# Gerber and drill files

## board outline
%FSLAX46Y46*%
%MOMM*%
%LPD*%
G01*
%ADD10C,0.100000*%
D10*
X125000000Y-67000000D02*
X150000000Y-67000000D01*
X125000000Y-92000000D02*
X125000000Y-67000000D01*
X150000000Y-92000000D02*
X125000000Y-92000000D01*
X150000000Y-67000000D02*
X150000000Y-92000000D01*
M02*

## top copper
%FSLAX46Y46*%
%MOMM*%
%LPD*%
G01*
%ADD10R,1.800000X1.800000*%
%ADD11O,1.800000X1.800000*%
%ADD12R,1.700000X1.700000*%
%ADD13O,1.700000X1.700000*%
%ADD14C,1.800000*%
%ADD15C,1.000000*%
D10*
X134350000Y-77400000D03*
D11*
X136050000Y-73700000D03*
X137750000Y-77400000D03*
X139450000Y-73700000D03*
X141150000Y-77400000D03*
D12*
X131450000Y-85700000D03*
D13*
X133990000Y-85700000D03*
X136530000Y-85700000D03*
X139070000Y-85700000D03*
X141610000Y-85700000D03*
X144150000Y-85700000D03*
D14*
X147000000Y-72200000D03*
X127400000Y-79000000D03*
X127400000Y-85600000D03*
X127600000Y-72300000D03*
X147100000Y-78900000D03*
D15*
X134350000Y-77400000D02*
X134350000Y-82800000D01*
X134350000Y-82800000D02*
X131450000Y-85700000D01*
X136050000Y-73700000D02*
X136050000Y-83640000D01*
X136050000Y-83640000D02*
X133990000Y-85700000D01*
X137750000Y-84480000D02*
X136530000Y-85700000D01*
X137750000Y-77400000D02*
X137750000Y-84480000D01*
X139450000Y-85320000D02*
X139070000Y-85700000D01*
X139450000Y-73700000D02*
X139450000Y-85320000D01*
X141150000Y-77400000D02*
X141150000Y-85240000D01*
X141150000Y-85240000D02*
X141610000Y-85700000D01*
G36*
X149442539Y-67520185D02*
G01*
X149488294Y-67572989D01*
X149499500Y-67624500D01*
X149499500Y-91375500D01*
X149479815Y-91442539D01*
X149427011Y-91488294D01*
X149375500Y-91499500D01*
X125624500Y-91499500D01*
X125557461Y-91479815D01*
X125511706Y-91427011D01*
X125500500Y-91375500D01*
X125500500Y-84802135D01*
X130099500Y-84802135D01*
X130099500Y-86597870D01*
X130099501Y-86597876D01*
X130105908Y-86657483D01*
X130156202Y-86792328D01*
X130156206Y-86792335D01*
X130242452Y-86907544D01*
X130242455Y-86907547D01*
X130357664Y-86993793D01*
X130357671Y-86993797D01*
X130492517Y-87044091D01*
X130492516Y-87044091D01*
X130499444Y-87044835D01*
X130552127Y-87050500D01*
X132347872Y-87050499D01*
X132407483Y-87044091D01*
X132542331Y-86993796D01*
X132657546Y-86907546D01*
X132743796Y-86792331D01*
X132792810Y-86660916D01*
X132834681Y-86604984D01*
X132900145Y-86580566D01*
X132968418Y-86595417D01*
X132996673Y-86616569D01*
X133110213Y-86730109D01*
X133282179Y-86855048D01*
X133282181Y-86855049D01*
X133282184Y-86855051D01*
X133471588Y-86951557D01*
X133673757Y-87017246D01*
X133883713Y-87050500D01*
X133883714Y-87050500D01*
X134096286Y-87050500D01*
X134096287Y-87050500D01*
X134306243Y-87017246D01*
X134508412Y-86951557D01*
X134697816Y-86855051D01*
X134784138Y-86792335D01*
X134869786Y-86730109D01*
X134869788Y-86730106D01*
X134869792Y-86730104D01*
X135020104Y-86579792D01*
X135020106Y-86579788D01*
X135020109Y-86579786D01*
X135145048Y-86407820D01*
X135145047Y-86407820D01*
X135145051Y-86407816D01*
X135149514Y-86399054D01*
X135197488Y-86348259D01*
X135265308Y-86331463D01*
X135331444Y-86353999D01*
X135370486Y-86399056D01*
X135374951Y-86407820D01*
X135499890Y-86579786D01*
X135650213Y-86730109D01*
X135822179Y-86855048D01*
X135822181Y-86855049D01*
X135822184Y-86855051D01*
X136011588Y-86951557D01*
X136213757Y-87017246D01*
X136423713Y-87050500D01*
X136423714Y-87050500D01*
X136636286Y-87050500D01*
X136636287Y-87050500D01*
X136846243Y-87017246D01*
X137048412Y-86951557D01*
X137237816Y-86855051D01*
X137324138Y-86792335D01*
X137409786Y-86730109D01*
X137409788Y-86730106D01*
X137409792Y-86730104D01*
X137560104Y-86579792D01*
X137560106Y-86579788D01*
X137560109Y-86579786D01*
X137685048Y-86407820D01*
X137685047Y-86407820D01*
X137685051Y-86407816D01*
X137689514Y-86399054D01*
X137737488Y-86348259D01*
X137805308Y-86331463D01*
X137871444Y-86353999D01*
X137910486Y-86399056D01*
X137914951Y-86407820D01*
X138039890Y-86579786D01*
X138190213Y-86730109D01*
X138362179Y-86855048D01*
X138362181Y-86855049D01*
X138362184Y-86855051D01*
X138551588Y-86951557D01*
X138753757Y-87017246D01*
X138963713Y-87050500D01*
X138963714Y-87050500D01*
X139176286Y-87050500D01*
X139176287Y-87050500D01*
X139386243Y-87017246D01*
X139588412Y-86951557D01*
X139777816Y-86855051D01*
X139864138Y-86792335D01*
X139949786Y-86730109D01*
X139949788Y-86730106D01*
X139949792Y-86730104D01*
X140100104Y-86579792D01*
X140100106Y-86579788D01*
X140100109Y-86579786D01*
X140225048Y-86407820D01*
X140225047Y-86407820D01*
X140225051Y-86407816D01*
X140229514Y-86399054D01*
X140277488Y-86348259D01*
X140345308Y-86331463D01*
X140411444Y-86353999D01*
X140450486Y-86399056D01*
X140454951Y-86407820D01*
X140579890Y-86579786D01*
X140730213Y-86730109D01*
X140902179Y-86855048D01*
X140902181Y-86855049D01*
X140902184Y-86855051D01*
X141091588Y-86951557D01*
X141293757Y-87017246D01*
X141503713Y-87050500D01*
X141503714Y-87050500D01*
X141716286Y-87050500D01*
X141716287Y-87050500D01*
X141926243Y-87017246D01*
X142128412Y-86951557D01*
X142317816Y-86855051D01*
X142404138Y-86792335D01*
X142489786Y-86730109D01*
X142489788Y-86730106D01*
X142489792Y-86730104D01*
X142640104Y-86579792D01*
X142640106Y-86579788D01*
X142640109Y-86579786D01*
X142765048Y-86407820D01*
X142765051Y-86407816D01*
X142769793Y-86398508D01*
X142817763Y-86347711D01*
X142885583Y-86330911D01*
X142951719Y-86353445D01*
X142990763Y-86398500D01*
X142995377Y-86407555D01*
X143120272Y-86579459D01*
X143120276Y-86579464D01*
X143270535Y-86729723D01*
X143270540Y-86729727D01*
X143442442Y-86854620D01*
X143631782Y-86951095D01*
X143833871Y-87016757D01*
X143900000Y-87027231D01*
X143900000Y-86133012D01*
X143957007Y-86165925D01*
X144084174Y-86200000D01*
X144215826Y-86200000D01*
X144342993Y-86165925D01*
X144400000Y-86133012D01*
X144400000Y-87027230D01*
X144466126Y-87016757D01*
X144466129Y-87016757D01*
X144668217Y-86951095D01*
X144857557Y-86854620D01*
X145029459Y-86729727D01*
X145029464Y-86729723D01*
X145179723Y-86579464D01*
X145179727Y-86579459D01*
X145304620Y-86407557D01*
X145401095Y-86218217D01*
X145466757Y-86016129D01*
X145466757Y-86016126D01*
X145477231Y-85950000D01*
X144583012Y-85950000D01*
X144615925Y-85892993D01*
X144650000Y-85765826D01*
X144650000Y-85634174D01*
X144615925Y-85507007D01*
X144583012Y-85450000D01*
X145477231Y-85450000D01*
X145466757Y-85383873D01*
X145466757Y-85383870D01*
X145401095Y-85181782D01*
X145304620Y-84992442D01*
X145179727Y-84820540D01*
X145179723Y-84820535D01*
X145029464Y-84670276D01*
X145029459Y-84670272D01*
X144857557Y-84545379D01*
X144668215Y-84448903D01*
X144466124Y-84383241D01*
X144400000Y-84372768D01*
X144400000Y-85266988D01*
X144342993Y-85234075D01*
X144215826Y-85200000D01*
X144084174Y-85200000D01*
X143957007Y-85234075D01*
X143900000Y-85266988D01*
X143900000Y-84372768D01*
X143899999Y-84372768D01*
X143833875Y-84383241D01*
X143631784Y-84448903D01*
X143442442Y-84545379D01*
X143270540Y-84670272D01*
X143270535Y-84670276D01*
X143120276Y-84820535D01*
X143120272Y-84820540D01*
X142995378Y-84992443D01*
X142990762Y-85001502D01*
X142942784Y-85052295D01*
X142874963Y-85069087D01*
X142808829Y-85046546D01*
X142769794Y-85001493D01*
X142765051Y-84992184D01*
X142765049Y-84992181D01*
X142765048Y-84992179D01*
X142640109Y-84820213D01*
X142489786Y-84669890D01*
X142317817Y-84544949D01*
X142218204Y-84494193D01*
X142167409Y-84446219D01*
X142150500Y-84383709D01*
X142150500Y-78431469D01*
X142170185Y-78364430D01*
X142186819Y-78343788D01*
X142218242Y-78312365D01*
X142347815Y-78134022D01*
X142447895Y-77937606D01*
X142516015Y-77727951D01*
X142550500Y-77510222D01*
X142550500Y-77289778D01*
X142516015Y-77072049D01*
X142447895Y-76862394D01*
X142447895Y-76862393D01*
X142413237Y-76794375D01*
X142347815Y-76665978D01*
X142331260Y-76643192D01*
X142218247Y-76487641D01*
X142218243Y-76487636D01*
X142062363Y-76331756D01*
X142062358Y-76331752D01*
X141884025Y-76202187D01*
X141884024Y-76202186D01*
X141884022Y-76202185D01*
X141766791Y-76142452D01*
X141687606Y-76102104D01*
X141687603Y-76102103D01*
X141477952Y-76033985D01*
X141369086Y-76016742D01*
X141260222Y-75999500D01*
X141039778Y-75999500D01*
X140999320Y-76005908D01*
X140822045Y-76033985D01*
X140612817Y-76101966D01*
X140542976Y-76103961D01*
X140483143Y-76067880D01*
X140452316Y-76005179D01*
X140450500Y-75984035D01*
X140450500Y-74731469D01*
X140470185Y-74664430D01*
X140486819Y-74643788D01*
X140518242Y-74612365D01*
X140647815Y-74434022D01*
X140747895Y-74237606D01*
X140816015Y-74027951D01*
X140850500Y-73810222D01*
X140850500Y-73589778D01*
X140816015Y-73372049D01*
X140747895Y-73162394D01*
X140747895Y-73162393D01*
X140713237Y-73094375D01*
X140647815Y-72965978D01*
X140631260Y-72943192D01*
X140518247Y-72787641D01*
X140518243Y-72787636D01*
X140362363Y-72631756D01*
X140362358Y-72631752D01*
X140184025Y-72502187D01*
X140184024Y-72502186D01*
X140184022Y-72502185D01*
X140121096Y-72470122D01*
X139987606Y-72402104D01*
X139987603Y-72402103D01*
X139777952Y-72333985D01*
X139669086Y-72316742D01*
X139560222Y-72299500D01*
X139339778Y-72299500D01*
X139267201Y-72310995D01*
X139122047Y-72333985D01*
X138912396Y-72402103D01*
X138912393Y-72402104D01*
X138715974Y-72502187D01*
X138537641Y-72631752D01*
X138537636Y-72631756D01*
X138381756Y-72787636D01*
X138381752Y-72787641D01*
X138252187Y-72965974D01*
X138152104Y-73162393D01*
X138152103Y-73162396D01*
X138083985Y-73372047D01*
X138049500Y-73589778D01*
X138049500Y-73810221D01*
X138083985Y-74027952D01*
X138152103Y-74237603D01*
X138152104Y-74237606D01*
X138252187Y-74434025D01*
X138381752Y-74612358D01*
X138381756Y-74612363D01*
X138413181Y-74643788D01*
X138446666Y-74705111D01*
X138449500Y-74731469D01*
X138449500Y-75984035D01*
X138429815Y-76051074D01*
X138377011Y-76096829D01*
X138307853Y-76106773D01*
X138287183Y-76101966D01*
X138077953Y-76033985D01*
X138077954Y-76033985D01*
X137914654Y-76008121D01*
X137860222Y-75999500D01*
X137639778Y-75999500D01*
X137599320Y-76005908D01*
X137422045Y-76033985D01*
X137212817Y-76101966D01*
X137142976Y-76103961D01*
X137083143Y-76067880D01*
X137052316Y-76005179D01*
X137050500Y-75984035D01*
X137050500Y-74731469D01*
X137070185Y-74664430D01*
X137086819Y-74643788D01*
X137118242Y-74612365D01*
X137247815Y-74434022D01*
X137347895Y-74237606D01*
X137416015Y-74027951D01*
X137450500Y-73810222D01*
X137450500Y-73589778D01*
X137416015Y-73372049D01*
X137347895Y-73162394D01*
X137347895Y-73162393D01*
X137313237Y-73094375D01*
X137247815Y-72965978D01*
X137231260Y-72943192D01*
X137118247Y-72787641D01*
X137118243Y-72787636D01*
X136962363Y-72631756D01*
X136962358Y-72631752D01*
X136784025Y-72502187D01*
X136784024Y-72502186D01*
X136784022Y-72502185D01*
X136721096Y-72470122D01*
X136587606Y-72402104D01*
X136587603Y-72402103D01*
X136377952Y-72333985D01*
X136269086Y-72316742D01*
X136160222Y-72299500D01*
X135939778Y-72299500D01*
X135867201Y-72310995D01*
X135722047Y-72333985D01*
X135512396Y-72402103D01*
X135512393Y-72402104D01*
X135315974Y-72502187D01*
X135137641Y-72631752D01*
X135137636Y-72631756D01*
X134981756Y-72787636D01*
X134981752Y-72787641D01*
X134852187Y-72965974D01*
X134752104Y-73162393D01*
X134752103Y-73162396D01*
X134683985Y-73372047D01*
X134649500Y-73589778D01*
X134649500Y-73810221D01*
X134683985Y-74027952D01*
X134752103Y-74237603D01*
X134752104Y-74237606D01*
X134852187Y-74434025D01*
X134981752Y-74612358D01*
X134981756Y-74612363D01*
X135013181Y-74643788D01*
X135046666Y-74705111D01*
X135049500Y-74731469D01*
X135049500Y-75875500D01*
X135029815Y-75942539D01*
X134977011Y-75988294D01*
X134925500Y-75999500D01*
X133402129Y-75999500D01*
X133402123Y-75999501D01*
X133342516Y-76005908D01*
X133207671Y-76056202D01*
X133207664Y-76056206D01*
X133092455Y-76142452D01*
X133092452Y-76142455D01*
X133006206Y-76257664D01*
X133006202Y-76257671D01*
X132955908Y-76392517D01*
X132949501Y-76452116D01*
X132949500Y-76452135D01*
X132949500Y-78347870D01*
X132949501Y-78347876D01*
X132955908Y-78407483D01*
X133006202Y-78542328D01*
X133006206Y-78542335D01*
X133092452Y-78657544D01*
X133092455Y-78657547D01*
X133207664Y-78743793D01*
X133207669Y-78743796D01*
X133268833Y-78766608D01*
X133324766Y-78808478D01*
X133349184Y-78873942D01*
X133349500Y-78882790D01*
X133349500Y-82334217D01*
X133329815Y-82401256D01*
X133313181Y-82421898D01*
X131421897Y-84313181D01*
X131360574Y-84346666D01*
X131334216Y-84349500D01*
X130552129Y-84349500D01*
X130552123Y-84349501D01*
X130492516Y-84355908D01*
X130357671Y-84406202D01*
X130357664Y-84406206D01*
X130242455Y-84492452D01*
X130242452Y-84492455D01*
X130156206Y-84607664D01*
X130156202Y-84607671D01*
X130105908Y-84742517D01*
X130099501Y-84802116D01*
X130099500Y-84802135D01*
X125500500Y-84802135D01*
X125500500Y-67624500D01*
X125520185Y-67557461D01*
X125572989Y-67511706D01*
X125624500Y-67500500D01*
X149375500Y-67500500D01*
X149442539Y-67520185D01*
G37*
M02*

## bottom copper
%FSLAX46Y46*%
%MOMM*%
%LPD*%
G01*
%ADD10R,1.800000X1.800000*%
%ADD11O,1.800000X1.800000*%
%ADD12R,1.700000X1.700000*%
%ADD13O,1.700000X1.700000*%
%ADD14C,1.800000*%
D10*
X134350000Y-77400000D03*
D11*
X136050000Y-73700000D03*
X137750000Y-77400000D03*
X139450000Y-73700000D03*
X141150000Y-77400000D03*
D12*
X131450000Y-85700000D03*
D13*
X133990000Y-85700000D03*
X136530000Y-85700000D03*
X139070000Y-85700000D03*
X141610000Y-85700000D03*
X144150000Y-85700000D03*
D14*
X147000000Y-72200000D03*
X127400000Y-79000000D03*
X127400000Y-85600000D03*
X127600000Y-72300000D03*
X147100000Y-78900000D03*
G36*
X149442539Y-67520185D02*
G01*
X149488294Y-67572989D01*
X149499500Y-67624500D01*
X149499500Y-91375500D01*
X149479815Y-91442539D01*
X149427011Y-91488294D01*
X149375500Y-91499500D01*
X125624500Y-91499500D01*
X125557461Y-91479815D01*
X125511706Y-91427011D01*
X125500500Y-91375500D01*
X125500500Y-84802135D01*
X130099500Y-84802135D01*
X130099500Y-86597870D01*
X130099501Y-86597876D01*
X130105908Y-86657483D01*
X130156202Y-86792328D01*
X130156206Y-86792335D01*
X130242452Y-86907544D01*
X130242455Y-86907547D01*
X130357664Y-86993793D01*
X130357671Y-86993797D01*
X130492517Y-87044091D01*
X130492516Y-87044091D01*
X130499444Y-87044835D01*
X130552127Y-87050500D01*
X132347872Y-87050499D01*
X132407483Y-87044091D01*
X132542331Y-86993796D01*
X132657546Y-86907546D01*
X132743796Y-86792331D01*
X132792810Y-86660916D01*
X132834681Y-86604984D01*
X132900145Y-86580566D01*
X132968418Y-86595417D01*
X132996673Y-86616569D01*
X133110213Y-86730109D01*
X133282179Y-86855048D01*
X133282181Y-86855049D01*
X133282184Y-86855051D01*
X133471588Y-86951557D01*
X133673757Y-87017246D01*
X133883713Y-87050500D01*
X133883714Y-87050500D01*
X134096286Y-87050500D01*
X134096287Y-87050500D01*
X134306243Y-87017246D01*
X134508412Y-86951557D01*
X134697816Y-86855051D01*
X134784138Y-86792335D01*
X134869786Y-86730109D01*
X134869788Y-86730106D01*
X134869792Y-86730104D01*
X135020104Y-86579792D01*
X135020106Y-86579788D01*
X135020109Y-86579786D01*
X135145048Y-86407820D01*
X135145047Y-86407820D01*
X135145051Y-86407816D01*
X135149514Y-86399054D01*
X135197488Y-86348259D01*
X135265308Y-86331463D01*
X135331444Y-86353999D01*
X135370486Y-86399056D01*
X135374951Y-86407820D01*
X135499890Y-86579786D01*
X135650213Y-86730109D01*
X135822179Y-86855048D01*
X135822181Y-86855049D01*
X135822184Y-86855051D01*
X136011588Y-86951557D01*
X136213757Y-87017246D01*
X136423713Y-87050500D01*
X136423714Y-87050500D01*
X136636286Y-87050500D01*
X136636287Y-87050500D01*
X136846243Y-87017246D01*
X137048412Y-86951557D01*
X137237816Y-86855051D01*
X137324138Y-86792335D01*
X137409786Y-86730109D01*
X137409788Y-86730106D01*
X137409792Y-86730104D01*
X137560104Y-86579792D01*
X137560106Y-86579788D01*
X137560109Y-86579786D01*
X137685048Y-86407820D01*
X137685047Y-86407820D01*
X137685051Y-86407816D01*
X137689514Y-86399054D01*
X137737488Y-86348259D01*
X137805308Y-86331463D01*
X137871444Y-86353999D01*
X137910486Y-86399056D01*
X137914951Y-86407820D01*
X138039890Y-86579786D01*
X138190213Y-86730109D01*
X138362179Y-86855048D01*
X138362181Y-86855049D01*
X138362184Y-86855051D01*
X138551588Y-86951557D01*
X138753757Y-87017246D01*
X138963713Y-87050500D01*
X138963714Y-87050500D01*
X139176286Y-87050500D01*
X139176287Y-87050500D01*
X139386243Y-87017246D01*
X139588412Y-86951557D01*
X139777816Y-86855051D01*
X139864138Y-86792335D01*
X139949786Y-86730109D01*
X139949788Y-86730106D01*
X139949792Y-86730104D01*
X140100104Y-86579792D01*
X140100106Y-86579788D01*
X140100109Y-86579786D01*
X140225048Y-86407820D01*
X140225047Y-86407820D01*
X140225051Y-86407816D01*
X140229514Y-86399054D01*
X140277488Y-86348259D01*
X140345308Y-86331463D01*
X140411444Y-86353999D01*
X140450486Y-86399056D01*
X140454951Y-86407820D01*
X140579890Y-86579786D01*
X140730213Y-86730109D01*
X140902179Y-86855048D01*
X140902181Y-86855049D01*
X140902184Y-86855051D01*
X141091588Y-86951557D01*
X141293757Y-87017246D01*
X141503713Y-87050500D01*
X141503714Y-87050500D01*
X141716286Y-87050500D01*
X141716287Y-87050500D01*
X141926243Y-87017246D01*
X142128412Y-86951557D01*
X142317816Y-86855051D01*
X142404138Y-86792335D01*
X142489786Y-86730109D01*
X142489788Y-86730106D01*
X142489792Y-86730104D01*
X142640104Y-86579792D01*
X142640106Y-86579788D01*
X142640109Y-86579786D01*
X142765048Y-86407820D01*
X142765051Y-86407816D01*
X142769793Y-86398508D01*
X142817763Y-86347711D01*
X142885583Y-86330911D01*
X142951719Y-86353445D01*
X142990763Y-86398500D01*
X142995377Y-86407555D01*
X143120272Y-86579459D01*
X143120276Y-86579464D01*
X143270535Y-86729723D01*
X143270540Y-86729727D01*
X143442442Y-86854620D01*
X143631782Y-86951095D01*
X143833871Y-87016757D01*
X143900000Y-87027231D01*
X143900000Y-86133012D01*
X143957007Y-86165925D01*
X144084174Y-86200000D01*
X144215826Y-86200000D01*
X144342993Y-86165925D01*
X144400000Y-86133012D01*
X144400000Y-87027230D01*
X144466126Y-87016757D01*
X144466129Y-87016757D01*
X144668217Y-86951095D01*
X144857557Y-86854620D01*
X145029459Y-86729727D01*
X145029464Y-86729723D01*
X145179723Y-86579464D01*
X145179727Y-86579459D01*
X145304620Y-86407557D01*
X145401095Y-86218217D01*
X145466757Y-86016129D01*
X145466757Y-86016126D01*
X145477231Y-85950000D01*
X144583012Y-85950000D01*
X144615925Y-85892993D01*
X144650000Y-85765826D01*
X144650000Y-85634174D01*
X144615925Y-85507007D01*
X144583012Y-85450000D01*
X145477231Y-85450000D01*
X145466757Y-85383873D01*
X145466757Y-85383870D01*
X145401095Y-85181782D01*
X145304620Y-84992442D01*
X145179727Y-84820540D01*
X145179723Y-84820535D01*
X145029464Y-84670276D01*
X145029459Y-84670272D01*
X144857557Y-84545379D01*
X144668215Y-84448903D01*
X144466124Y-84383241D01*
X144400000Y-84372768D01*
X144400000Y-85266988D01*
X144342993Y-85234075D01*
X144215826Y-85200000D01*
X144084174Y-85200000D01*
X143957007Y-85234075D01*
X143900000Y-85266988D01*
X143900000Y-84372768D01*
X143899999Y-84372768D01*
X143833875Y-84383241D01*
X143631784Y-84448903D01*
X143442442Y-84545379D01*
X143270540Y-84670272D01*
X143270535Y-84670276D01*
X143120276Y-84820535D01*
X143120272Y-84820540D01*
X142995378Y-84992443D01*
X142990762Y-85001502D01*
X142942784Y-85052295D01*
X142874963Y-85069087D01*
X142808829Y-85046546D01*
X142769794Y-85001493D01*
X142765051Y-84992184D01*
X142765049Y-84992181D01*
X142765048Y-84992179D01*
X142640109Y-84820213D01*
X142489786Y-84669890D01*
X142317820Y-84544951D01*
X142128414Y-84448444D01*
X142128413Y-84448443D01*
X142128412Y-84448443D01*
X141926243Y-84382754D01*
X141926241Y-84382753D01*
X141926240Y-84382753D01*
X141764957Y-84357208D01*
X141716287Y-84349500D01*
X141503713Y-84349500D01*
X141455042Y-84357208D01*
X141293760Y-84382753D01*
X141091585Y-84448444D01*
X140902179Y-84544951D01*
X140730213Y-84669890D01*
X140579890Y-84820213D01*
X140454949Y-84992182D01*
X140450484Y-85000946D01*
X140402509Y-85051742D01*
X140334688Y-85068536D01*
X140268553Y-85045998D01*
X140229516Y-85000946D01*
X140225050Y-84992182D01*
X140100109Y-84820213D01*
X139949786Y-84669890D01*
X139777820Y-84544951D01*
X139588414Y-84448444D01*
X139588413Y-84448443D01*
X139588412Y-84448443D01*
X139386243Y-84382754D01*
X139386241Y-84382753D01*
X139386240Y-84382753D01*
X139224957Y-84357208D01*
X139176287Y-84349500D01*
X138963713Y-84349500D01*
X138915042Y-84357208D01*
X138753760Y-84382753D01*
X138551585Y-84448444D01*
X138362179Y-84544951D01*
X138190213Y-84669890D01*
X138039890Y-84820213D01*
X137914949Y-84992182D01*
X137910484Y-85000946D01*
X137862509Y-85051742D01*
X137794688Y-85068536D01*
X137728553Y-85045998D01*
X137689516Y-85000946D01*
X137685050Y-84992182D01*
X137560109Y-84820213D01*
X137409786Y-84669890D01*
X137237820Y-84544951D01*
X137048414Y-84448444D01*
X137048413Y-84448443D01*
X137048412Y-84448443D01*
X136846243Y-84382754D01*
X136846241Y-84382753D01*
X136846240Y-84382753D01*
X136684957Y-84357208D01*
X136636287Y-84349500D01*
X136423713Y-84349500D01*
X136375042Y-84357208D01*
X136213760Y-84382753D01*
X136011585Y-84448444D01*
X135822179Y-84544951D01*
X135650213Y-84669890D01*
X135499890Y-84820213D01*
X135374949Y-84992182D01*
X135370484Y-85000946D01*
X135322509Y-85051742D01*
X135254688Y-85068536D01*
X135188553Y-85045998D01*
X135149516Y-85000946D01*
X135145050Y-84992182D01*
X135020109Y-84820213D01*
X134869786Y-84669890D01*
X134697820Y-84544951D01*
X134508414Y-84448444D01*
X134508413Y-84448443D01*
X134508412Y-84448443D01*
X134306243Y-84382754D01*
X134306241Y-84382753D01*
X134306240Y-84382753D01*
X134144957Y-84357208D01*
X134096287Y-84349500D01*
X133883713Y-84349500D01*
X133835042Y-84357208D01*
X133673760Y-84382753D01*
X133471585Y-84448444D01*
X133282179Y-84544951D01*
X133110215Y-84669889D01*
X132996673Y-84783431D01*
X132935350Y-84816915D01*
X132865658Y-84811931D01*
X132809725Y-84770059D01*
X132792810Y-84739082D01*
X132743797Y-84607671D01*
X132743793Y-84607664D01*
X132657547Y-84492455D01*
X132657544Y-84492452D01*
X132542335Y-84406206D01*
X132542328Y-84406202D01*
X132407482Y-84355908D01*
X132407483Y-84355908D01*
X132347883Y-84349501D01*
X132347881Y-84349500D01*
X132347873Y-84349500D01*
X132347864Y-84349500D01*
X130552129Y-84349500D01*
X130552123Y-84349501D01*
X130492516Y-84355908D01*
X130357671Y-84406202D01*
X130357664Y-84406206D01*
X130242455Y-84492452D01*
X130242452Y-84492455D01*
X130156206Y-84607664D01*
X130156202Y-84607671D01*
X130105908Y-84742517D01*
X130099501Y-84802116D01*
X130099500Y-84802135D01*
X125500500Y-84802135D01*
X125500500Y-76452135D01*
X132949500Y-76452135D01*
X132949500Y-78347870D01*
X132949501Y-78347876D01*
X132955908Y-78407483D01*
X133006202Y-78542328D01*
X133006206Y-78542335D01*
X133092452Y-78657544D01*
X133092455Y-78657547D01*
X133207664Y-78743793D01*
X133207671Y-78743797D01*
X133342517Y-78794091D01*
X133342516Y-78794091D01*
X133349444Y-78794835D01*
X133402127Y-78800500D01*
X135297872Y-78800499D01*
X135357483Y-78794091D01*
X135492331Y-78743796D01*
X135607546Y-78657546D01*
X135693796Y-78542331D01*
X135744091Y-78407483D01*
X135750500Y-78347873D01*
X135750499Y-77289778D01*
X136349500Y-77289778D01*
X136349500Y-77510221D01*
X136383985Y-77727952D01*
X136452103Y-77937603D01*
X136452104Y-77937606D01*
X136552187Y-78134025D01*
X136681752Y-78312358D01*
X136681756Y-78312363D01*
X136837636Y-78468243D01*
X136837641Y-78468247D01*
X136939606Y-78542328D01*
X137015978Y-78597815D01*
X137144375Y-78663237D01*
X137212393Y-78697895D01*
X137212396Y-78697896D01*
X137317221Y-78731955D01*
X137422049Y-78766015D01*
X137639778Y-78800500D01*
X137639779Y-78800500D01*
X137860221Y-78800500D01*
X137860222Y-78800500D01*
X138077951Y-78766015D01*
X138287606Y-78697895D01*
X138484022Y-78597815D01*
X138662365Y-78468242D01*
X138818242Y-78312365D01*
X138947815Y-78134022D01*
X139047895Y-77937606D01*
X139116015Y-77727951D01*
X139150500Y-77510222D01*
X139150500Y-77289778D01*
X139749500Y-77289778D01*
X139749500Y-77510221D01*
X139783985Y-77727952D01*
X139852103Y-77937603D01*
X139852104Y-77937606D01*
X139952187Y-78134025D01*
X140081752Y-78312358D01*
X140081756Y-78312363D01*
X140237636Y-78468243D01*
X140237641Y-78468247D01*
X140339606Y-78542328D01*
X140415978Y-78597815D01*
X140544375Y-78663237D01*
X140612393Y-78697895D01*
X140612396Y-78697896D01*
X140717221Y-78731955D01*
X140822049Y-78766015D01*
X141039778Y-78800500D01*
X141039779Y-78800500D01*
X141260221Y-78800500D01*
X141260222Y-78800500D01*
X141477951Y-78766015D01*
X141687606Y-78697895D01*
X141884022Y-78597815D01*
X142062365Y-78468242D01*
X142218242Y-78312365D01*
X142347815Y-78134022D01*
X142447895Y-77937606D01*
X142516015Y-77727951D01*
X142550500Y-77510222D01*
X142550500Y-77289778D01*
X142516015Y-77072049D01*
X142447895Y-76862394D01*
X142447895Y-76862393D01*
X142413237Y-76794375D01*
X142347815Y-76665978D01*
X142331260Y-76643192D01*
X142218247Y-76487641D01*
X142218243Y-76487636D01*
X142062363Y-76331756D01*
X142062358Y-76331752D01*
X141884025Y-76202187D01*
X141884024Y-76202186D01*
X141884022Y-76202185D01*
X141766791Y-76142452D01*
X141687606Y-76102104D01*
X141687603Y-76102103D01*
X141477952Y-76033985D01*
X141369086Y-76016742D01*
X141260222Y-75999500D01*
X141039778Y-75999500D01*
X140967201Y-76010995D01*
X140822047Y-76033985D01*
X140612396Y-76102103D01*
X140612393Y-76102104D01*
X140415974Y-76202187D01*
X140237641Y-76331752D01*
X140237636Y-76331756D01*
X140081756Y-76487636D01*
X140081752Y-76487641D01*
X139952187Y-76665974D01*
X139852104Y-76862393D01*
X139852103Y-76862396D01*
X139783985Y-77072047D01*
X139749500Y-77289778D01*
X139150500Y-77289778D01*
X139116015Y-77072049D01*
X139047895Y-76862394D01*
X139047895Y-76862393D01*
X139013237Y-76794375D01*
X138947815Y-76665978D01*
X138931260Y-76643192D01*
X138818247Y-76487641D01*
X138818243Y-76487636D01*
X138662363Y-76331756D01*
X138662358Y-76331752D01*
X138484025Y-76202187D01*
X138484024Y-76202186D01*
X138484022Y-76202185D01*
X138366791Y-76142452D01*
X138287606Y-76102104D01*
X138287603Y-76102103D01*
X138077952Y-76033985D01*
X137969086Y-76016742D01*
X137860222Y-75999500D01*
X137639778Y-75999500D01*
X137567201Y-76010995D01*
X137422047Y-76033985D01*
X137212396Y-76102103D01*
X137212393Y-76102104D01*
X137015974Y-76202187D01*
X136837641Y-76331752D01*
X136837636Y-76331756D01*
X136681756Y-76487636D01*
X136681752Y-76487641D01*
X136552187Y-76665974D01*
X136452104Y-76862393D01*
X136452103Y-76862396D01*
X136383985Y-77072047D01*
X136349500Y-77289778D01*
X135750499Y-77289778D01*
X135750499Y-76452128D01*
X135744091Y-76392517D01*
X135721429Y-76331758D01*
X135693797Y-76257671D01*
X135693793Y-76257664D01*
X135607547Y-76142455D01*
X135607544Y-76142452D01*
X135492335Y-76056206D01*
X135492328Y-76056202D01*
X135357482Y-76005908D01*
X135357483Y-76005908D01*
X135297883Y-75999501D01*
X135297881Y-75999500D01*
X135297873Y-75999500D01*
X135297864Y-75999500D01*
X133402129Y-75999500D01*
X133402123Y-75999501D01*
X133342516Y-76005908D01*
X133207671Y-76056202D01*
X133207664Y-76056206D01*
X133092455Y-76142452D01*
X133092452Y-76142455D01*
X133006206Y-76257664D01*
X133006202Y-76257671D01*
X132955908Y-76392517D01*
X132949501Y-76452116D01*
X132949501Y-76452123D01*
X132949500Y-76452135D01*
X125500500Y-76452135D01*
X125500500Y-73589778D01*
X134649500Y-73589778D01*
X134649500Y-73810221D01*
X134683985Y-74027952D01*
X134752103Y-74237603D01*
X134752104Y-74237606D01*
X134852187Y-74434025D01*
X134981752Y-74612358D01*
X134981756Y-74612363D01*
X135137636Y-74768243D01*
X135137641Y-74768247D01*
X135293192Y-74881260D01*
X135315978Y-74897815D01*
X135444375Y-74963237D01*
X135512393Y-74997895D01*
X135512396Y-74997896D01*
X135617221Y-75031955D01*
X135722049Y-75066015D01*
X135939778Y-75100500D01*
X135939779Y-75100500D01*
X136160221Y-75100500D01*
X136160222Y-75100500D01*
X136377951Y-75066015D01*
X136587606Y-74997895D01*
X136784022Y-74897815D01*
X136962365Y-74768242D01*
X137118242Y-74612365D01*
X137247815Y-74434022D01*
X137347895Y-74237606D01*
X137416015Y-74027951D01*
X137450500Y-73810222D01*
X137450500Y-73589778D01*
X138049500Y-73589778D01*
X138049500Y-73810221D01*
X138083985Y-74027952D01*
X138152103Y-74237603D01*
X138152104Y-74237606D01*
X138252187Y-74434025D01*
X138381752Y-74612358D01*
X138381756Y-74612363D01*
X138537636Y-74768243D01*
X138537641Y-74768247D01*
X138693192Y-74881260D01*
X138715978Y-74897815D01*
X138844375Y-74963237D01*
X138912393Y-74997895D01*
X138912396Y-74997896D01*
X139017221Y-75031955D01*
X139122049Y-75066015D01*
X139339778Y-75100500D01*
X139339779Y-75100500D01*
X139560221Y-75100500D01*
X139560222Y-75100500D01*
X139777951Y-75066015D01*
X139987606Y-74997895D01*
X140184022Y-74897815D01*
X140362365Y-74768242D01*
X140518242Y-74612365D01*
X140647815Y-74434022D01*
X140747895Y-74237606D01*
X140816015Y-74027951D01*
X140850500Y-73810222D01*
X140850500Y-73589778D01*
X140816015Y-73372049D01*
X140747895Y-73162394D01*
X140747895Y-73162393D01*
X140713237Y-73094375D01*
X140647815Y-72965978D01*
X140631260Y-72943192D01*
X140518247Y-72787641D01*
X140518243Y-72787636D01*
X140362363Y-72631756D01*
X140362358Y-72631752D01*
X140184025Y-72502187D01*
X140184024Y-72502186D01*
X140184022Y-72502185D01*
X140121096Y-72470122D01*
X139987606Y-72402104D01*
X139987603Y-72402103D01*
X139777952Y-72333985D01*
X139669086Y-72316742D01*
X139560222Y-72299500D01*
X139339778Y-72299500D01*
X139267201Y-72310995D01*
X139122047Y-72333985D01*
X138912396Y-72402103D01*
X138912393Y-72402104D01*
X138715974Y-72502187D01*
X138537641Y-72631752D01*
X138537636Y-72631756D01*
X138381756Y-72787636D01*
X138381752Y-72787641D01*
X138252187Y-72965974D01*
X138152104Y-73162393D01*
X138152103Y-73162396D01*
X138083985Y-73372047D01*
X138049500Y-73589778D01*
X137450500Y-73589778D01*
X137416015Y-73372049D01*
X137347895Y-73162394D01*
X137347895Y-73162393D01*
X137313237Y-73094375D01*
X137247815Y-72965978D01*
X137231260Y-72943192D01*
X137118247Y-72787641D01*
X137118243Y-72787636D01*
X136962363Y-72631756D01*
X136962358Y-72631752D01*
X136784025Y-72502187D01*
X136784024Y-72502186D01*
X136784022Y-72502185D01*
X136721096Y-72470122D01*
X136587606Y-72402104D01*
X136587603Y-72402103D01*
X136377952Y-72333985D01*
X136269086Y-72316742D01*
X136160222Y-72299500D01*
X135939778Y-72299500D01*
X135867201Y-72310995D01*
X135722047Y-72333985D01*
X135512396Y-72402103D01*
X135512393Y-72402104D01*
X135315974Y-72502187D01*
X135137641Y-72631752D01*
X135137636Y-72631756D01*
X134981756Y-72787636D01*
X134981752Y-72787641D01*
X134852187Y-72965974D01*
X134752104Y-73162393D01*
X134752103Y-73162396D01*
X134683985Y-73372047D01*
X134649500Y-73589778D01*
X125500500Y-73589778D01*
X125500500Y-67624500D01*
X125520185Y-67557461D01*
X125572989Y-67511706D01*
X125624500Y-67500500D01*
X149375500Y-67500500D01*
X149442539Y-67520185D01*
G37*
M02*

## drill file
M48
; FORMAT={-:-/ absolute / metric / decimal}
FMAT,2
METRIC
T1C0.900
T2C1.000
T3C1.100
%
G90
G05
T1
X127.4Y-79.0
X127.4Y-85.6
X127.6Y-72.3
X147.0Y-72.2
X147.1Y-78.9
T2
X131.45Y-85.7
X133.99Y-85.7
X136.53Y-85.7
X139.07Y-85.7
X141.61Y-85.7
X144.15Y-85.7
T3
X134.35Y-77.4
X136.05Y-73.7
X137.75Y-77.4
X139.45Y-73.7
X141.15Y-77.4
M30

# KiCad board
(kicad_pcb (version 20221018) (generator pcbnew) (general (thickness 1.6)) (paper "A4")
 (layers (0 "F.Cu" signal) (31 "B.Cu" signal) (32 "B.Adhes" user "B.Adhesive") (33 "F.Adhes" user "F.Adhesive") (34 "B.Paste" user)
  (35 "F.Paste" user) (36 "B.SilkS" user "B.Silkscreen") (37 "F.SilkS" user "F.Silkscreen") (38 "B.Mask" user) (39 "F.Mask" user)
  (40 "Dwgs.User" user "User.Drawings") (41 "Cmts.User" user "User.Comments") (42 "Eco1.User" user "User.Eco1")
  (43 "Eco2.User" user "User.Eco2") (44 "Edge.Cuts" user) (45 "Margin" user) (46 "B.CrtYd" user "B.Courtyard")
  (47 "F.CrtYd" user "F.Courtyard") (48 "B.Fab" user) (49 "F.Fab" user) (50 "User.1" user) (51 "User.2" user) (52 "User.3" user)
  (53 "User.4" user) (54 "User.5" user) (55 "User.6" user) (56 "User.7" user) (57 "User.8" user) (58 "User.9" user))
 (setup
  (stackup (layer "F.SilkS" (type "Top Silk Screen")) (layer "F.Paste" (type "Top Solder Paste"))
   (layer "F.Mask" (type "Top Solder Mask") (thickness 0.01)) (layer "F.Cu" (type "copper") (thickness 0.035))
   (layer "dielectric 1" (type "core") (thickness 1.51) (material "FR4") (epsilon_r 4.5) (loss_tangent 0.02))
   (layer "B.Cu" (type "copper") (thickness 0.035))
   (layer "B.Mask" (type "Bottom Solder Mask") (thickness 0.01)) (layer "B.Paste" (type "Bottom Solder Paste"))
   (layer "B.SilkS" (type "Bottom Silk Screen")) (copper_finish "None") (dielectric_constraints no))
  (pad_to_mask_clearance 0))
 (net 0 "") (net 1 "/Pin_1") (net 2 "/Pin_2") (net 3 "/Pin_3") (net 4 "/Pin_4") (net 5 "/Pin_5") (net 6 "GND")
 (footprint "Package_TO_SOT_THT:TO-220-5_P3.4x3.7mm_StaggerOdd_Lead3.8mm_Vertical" (layer "F.Cu") (at 134.35 77.4)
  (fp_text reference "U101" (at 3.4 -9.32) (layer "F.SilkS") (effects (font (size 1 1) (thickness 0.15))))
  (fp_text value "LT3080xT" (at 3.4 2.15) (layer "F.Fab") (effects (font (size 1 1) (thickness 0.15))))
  (pad "1" thru_hole rect (at 0 0) (size 1.8 1.8) (drill 1.1) (layers "*.Cu" "*.Mask") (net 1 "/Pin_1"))
  (pad "2" thru_hole oval (at 1.7 -3.7) (size 1.8 1.8) (drill 1.1) (layers "*.Cu" "*.Mask") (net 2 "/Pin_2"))
  (pad "3" thru_hole oval (at 3.4 0) (size 1.8 1.8) (drill 1.1) (layers "*.Cu" "*.Mask") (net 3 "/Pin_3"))
  (pad "4" thru_hole oval (at 5.1 -3.7) (size 1.8 1.8) (drill 1.1) (layers "*.Cu" "*.Mask") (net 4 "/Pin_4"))
  (pad "5" thru_hole oval (at 6.8 0) (size 1.8 1.8) (drill 1.1) (layers "*.Cu" "*.Mask") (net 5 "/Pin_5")))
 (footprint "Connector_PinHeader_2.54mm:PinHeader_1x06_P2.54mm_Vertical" (layer "B.Cu") (at 131.45 85.7 -90)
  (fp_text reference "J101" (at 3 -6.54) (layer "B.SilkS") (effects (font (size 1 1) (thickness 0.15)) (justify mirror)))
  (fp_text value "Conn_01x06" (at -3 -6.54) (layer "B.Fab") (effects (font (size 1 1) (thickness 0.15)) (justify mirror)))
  (pad "1" thru_hole rect (at 0 0 270) (size 1.7 1.7) (drill 1) (layers "*.Cu" "*.Mask") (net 1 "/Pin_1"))
  (pad "2" thru_hole oval (at 0 -2.54 270) (size 1.7 1.7) (drill 1) (layers "*.Cu" "*.Mask") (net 2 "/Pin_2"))
  (pad "3" thru_hole oval (at 0 -5.08 270) (size 1.7 1.7) (drill 1) (layers "*.Cu" "*.Mask") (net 3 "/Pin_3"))
  (pad "4" thru_hole oval (at 0 -7.62 270) (size 1.7 1.7) (drill 1) (layers "*.Cu" "*.Mask") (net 4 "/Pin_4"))
  (pad "5" thru_hole oval (at 0 -10.16 270) (size 1.7 1.7) (drill 1) (layers "*.Cu" "*.Mask") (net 5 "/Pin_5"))
  (pad "6" thru_hole oval (at 0 -12.7 270) (size 1.7 1.7) (drill 1) (layers "*.Cu" "*.Mask") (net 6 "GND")))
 (gr_line (start 125 67) (end 150 67) (stroke (width 0.1) (type default)) (layer "Edge.Cuts"))
 (gr_line (start 125 92) (end 125 67) (stroke (width 0.1) (type default)) (layer "Edge.Cuts"))
 (gr_line (start 150 92) (end 125 92) (stroke (width 0.1) (type default)) (layer "Edge.Cuts"))
 (gr_line (start 150 67) (end 150 92) (stroke (width 0.1) (type default)) (layer "Edge.Cuts"))
 (segment (start 134.35 77.4) (end 134.35 82.8) (width 1) (layer "F.Cu") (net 1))
 (segment (start 134.35 82.8) (end 131.45 85.7) (width 1) (layer "F.Cu") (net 1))
 (segment (start 136.05 73.7) (end 136.05 83.64) (width 1) (layer "F.Cu") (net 2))
 (segment (start 136.05 83.64) (end 133.99 85.7) (width 1) (layer "F.Cu") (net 2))
 (segment (start 137.75 84.48) (end 136.53 85.7) (width 1) (layer "F.Cu") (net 3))
 (segment (start 137.75 77.4) (end 137.75 84.48) (width 1) (layer "F.Cu") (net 3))
 (segment (start 139.45 85.32) (end 139.07 85.7) (width 1) (layer "F.Cu") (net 4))
 (segment (start 139.45 73.7) (end 139.45 85.32) (width 1) (layer "F.Cu") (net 4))
 (segment (start 141.15 77.4) (end 141.15 85.24) (width 1) (layer "F.Cu") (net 5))
 (segment (start 141.15 85.24) (end 141.61 85.7) (width 1) (layer "F.Cu") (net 5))
 (via (at 147 72.2) (size 1.8) (drill 0.9) (layers "F.Cu" "B.Cu") (free) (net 6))
 (via (at 127.4 79) (size 1.8) (drill 0.9) (layers "F.Cu" "B.Cu") (free) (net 6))
 (via (at 127.4 85.6) (size 1.8) (drill 0.9) (layers "F.Cu" "B.Cu") (free) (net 6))
 (via (at 127.6 72.3) (size 1.8) (drill 0.9) (layers "F.Cu" "B.Cu") (free) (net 6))
 (via (at 147.1 78.9) (size 1.8) (drill 0.9) (layers "F.Cu" "B.Cu") (free) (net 6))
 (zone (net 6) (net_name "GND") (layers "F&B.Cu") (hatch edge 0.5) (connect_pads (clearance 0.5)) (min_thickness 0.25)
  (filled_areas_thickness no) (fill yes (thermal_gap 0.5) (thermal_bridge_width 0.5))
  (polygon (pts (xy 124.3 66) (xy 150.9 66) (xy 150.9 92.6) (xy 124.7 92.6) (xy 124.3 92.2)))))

